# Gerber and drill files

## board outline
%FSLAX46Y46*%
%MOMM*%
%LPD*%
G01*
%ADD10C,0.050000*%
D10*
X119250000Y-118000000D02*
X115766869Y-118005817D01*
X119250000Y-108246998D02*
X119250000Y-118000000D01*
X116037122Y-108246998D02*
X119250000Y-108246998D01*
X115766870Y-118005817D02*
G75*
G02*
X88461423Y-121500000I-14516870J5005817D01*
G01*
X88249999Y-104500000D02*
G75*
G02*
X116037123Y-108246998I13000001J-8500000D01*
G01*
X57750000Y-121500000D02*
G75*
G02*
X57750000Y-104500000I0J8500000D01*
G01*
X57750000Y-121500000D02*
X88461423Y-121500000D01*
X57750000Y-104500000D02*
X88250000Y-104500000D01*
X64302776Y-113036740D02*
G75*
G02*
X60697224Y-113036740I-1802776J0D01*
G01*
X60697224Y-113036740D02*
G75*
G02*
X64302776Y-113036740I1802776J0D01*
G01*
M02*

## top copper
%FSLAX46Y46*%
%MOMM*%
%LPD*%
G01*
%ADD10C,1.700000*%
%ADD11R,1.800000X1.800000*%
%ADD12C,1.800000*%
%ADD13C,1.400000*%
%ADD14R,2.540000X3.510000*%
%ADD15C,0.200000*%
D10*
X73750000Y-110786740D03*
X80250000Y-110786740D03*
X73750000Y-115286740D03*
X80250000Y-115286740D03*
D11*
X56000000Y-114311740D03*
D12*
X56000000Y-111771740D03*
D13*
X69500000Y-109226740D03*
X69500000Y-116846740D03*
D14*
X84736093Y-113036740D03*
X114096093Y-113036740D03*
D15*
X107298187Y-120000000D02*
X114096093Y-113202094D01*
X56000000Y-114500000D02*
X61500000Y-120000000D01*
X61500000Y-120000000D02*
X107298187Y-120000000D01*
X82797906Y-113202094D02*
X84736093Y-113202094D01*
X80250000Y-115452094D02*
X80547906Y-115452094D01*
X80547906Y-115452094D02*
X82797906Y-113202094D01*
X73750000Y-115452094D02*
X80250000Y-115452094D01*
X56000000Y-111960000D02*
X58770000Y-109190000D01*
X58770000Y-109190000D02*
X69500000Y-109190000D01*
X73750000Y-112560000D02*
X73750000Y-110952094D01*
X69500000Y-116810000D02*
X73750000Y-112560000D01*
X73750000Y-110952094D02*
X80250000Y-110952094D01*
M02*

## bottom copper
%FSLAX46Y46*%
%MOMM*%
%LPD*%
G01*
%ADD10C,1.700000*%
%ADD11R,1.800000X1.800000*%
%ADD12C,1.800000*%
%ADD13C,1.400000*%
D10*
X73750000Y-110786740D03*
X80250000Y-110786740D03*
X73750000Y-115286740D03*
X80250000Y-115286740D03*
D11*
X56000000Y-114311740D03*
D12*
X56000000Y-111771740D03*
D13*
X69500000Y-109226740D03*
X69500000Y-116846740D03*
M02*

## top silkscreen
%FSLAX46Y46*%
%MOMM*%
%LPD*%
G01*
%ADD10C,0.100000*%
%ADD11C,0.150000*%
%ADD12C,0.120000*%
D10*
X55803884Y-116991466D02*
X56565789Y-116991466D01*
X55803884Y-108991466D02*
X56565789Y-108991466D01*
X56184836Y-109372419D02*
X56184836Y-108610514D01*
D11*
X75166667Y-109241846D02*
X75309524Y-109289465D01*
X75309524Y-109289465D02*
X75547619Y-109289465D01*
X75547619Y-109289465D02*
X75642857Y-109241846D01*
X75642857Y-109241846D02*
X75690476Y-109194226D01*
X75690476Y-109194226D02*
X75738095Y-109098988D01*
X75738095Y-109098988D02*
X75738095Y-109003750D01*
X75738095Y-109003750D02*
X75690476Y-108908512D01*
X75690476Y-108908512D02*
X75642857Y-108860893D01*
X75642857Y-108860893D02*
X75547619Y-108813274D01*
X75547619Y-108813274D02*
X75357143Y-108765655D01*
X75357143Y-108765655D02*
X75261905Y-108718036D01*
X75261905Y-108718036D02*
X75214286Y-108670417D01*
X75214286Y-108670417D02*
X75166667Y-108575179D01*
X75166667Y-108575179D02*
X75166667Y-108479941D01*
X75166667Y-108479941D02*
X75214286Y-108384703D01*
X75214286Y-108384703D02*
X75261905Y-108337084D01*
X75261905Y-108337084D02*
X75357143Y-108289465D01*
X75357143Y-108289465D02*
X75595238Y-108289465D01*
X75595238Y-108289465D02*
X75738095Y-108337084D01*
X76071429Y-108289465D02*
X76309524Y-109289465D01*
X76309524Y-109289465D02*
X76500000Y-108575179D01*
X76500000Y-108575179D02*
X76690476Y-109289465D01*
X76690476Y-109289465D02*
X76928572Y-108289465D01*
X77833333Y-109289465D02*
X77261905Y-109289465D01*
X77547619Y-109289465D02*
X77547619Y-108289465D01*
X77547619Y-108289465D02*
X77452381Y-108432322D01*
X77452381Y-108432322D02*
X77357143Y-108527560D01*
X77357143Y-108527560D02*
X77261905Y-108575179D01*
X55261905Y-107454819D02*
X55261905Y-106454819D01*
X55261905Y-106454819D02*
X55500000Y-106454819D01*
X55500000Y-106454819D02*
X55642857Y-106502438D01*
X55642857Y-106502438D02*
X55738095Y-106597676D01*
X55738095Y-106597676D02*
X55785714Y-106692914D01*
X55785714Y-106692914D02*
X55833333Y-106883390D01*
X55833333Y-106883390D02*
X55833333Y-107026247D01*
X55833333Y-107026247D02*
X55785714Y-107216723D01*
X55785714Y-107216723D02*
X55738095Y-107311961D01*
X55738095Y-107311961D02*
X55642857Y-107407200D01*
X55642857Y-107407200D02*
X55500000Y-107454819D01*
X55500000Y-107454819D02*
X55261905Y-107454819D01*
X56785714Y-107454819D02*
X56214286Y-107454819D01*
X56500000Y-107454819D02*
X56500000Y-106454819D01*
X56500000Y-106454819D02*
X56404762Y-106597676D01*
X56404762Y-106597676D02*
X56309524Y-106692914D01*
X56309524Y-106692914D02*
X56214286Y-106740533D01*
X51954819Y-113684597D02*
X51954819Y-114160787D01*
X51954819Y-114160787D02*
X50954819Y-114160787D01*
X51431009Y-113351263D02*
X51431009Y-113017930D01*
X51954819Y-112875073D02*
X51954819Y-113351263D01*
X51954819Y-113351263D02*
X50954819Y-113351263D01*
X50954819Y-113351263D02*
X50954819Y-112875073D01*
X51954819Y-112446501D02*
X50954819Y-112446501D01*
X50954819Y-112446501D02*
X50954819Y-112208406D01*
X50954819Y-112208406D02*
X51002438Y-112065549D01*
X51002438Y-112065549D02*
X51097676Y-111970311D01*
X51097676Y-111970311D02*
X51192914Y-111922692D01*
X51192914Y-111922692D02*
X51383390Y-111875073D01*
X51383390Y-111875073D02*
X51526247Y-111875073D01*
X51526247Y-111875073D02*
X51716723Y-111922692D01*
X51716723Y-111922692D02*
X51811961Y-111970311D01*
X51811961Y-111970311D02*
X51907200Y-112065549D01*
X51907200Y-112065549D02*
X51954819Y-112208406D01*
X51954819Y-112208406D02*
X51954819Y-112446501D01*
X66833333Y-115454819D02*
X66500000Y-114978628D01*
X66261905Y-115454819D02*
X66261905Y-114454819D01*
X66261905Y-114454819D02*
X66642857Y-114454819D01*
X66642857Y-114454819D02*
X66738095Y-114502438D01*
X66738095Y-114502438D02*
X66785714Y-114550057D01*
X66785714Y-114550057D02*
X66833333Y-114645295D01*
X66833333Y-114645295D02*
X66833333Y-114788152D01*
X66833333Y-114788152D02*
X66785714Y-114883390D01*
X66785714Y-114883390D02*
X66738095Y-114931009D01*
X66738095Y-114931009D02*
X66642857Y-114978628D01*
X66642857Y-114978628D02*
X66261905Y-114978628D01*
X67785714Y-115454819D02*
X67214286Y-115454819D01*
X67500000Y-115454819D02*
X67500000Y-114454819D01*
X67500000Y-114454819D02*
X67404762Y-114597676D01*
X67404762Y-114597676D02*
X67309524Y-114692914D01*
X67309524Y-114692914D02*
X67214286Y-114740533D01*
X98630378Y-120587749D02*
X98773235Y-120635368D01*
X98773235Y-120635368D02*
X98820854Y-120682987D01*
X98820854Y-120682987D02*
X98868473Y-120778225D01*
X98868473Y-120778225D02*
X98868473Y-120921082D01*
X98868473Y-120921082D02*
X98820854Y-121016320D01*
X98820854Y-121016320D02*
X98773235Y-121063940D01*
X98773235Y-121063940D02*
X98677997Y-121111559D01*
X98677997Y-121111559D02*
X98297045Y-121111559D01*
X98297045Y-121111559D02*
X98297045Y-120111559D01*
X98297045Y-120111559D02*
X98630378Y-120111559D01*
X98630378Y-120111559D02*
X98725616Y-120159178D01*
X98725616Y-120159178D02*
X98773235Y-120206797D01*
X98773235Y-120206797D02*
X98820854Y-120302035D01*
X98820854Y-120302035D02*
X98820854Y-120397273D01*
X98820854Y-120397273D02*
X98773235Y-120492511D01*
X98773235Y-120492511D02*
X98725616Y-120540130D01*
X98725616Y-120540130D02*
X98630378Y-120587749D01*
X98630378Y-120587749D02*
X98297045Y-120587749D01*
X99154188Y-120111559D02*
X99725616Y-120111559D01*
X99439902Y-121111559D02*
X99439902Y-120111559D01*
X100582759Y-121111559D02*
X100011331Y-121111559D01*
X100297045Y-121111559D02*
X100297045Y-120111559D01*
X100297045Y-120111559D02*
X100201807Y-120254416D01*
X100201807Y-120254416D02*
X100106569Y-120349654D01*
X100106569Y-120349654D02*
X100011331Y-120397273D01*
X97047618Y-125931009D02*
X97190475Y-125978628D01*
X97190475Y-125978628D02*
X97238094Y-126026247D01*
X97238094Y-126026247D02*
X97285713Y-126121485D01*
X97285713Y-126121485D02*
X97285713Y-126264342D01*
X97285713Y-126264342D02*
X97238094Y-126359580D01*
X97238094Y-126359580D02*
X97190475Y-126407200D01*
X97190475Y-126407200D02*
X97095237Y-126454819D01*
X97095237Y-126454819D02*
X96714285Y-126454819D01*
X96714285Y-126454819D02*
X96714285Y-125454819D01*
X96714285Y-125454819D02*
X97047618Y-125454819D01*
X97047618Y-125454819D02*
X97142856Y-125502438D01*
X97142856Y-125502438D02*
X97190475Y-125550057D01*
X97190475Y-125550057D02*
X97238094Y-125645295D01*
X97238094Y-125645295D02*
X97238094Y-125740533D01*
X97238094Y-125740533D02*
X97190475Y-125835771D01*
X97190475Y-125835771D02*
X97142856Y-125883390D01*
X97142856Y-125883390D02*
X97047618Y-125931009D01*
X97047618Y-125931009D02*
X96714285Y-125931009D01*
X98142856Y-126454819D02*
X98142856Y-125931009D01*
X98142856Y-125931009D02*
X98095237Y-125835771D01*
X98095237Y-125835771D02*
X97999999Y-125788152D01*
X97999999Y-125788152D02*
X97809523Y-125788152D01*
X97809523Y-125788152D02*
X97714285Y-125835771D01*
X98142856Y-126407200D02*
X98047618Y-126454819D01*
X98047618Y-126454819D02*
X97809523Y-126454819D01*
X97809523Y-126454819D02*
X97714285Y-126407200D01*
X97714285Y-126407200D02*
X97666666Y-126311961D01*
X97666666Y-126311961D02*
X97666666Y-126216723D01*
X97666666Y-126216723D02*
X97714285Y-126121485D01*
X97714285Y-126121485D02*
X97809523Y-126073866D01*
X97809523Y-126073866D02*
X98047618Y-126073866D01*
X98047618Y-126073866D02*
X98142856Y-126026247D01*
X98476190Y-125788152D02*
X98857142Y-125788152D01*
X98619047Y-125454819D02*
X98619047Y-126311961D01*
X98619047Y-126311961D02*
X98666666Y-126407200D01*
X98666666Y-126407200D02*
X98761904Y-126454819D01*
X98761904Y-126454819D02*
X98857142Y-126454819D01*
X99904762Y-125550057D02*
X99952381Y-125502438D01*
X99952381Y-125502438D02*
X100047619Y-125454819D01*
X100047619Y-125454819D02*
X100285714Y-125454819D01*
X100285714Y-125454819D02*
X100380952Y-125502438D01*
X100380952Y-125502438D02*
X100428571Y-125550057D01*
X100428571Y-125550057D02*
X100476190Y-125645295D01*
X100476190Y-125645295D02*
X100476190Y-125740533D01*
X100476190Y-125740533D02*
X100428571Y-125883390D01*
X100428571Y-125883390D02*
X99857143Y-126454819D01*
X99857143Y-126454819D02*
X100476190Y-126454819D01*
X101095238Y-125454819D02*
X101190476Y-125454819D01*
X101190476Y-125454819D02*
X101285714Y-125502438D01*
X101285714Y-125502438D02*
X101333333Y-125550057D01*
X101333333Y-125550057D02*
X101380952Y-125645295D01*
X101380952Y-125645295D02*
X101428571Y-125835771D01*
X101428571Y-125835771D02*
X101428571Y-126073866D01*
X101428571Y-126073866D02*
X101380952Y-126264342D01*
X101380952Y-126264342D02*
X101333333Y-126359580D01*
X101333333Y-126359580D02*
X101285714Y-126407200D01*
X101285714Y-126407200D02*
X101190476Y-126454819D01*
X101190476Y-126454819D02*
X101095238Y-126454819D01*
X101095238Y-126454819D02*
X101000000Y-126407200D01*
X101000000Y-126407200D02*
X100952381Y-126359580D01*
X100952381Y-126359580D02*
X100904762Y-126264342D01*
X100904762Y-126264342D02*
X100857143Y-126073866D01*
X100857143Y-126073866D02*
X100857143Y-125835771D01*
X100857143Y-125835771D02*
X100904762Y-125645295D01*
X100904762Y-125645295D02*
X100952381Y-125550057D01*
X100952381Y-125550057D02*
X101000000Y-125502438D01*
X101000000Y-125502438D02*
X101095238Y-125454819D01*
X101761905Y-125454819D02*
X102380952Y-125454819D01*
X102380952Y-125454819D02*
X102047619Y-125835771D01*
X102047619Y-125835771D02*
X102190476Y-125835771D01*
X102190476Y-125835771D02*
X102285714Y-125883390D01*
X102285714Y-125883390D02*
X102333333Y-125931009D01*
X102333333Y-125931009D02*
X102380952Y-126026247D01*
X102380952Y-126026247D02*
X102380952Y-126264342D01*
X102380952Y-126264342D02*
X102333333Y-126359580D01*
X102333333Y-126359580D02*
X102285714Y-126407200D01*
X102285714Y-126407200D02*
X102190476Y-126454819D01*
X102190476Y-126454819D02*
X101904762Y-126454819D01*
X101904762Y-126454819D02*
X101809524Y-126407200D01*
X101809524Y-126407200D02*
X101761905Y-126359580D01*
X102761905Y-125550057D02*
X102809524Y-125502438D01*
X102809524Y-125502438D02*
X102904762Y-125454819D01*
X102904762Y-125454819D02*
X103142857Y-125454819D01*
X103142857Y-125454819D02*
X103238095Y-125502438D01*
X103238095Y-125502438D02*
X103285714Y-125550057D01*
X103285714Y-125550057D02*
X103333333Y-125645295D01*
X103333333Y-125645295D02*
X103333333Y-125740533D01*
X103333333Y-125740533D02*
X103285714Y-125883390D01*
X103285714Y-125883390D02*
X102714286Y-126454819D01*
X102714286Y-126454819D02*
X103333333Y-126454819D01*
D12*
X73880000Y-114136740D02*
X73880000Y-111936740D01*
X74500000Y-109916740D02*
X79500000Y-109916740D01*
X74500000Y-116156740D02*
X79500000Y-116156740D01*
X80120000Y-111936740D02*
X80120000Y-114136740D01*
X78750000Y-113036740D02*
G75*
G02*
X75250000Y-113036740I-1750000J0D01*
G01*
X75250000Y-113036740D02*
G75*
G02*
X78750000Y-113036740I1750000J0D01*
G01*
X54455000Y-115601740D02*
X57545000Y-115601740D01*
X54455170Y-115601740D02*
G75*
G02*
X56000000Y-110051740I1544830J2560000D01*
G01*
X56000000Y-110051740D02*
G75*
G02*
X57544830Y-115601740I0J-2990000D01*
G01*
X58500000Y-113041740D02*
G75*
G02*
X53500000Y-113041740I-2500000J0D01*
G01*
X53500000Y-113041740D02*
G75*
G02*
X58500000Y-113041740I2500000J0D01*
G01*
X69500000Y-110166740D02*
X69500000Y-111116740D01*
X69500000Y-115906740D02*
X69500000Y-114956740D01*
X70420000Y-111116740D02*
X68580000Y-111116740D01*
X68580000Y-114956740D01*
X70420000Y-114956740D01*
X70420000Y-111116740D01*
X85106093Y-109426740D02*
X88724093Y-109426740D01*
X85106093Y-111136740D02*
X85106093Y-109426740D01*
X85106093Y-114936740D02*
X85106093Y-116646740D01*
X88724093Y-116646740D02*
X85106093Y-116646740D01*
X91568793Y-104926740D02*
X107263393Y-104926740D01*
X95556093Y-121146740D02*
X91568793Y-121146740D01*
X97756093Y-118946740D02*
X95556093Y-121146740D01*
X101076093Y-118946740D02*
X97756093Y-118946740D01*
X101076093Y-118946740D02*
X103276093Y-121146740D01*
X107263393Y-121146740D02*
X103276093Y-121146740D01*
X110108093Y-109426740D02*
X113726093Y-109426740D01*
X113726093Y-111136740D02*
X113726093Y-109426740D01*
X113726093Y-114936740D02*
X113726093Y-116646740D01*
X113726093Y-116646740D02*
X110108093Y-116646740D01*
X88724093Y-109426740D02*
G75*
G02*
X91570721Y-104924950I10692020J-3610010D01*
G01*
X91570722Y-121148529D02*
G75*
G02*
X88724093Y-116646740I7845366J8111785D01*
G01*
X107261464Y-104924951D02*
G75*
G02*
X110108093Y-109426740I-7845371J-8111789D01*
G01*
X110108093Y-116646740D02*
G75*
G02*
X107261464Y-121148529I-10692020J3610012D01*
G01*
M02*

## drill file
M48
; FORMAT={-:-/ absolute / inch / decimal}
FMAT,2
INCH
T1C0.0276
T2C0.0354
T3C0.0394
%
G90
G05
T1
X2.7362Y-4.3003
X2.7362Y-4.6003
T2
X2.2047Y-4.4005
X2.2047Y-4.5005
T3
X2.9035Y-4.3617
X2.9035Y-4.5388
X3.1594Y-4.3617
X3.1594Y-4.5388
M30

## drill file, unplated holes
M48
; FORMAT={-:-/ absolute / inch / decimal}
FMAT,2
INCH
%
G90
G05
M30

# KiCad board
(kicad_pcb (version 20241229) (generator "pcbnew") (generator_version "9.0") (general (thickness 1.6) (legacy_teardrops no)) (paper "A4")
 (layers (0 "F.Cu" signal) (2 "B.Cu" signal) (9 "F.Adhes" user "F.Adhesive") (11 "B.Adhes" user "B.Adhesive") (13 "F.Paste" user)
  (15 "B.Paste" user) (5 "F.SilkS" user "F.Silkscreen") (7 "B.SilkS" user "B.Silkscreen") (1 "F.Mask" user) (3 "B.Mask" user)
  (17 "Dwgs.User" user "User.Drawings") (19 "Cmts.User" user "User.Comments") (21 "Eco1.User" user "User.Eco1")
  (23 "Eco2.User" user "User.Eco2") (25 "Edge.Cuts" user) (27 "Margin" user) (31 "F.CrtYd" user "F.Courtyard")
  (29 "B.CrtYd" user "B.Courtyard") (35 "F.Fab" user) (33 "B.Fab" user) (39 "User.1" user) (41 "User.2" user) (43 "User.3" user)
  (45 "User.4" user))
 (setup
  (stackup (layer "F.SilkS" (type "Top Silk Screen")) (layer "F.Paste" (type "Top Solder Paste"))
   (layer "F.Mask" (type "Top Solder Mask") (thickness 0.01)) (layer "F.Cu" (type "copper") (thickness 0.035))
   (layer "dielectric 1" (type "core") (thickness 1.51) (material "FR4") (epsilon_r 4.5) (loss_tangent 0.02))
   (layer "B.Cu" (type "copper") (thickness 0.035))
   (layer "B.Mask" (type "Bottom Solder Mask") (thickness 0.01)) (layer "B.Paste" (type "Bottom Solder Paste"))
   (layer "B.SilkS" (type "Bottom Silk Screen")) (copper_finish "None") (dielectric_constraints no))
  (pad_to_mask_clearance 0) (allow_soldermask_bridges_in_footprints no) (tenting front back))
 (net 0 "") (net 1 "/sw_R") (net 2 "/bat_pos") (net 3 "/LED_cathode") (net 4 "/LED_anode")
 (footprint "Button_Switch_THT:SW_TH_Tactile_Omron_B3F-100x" (layer "F.Cu") (at 73.75 110.78674)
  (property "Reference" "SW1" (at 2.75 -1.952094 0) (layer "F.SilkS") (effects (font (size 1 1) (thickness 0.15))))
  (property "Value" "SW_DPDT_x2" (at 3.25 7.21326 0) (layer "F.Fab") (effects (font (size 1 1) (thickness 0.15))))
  (fp_line (start 0.13 3.35) (end 0.13 1.15) (stroke (width 0.12) (type solid)) (layer "F.SilkS"))
  (fp_line (start 0.75 -0.87) (end 5.75 -0.87) (stroke (width 0.12) (type solid)) (layer "F.SilkS"))
  (fp_line (start 0.75 5.37) (end 5.75 5.37) (stroke (width 0.12) (type solid)) (layer "F.SilkS"))
  (fp_line (start 6.37 1.15) (end 6.37 3.35) (stroke (width 0.12) (type solid)) (layer "F.SilkS"))
  (fp_circle (center 3.25 2.25) (end 5 2.25) (stroke (width 0.12) (type solid)) (fill no) (layer "F.SilkS"))
  (pad "1" thru_hole circle (at 0 0) (size 1.7 1.7) (drill 1) (layers "*.Cu" "*.Mask") (remove_unused_layers no) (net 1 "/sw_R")
   (thermal_bridge_angle 90))
  (pad "1" thru_hole circle (at 6.5 0) (size 1.7 1.7) (drill 1) (layers "*.Cu" "*.Mask") (remove_unused_layers no) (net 1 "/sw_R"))
  (pad "2" thru_hole circle (at 0 4.5) (size 1.7 1.7) (drill 1) (layers "*.Cu" "*.Mask") (remove_unused_layers no) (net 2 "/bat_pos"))
  (pad "2" thru_hole circle (at 6.5 4.5) (size 1.7 1.7) (drill 1) (layers "*.Cu" "*.Mask") (remove_unused_layers no) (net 2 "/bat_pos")))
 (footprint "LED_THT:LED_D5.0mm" (layer "F.Cu") (at 56 114.31174 90)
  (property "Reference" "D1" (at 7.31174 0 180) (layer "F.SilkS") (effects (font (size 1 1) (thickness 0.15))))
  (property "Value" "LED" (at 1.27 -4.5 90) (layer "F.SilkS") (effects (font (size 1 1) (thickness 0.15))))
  (fp_line (start -1.29 -1.545) (end -1.29 1.545) (stroke (width 0.12) (type solid)) (layer "F.SilkS"))
  (fp_arc (start -1.29 -1.54483) (mid 2.071779 -2.880495) (end 4.26 0) (stroke (width 0.12) (type solid)) (layer "F.SilkS"))
  (fp_arc (start 4.26 0) (mid 2.071779 2.880495) (end -1.29 1.54483) (stroke (width 0.12) (type solid)) (layer "F.SilkS"))
  (fp_circle (center 1.27 0) (end 3.77 0) (stroke (width 0.12) (type solid)) (fill no) (layer "F.SilkS"))
  (pad "1" thru_hole rect (at 0 0 90) (size 1.8 1.8) (drill 0.9) (layers "*.Cu" "*.Mask") (remove_unused_layers no) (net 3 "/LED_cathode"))
  (pad "2" thru_hole circle (at 2.54 0 90) (size 1.8 1.8) (drill 0.9) (layers "*.Cu" "*.Mask") (remove_unused_layers no)
   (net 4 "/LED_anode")))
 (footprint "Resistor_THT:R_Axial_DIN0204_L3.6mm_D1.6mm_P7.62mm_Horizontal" (layer "F.Cu") (at 69.5 109.22674 -90)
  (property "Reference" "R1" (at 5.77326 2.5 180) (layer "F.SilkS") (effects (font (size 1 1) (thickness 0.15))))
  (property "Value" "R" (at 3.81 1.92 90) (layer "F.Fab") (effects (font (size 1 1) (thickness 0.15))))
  (fp_line (start 0.94 0) (end 1.89 0) (stroke (width 0.12) (type solid)) (layer "F.SilkS"))
  (fp_line (start 6.68 0) (end 5.73 0) (stroke (width 0.12) (type solid)) (layer "F.SilkS"))
  (fp_rect (start 1.89 -0.92) (end 5.73 0.92) (stroke (width 0.12) (type solid)) (fill no) (layer "F.SilkS"))
  (pad "1" thru_hole circle (at 0 0 270) (size 1.4 1.4) (drill 0.7) (layers "*.Cu" "*.Mask") (remove_unused_layers no) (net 4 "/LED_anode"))
  (pad "2" thru_hole circle (at 7.62 0 270) (size 1.4 1.4) (drill 0.7) (layers "*.Cu" "*.Mask") (remove_unused_layers no) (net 1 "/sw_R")))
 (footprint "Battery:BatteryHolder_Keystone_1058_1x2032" (layer "F.Cu") (at 99.416093 113.03674)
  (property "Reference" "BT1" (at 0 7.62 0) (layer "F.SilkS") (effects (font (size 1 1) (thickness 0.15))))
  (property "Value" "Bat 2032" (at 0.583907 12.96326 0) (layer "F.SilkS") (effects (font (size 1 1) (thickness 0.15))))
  (fp_line (start -14.31 -3.61) (end -10.692 -3.61) (stroke (width 0.12) (type solid)) (layer "F.SilkS"))
  (fp_line (start -14.31 -1.9) (end -14.31 -3.61) (stroke (width 0.12) (type solid)) (layer "F.SilkS"))
  (fp_line (start -14.31 1.9) (end -14.31 3.61) (stroke (width 0.12) (type solid)) (layer "F.SilkS"))
  (fp_line (start -10.692 3.61) (end -14.31 3.61) (stroke (width 0.12) (type solid)) (layer "F.SilkS"))
  (fp_line (start -7.8473 -8.11) (end 7.8473 -8.11) (stroke (width 0.12) (type solid)) (layer "F.SilkS"))
  (fp_line (start -3.86 8.11) (end -7.8473 8.11) (stroke (width 0.12) (type solid)) (layer "F.SilkS"))
  (fp_line (start -1.66 5.91) (end -3.86 8.11) (stroke (width 0.12) (type solid)) (layer "F.SilkS"))
  (fp_line (start 1.66 5.91) (end -1.66 5.91) (stroke (width 0.12) (type solid)) (layer "F.SilkS"))
  (fp_line (start 1.66 5.91) (end 3.86 8.11) (stroke (width 0.12) (type solid)) (layer "F.SilkS"))
  (fp_line (start 7.8473 8.11) (end 3.86 8.11) (stroke (width 0.12) (type solid)) (layer "F.SilkS"))
  (fp_line (start 10.692 -3.61) (end 14.31 -3.61) (stroke (width 0.12) (type solid)) (layer "F.SilkS"))
  (fp_line (start 14.31 -1.9) (end 14.31 -3.61) (stroke (width 0.12) (type solid)) (layer "F.SilkS"))
  (fp_line (start 14.31 1.9) (end 14.31 3.61) (stroke (width 0.12) (type solid)) (layer "F.SilkS"))
  (fp_line (start 14.31 3.61) (end 10.692 3.61) (stroke (width 0.12) (type solid)) (layer "F.SilkS"))
  (fp_arc (start -10.692 -3.61) (mid -9.538084 -6.031244) (end -7.845371 -8.111789) (stroke (width 0.12) (type solid)) (layer "F.SilkS"))
  (fp_arc (start -7.845371 8.111789) (mid -9.538085 6.031244) (end -10.692 3.61) (stroke (width 0.12) (type solid)) (layer "F.SilkS"))
  (fp_arc (start 7.845371 -8.111789) (mid 9.538085 -6.031244) (end 10.692 -3.61) (stroke (width 0.12) (type solid)) (layer "F.SilkS"))
  (fp_arc (start 10.692 3.61) (mid 9.538084 6.031244) (end 7.845371 8.111789) (stroke (width 0.12) (type solid)) (layer "F.SilkS"))
  (pad "1" smd rect (at -14.68 0) (size 2.54 3.51) (layers "F.Cu" "F.Mask" "F.Paste") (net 2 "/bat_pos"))
  (pad "2" smd rect (at 14.68 0) (size 2.54 3.51) (layers "F.Cu" "F.Mask" "F.Paste") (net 3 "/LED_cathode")))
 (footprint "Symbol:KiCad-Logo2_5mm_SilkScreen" (layer "B.Cu") (at 99 112.5 180)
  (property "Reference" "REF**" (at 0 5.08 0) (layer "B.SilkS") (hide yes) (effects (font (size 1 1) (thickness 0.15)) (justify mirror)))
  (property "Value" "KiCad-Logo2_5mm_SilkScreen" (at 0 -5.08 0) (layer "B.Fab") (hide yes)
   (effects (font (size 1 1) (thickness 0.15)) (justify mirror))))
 (gr_line (start 116.037122 108.246998) (end 119.25 108.246998) (stroke (width 0.05) (type default)) (locked yes) (layer "Edge.Cuts"))
 (gr_arc (start 88.249999 104.5) (mid 103.32568 97.607093) (end 116.037122 108.246998) (stroke (width 0.05) (type default)) (locked yes)
  (layer "Edge.Cuts"))
 (gr_line (start 57.75 121.5) (end 88.461423 121.5) (stroke (width 0.05) (type default)) (locked yes) (layer "Edge.Cuts"))
 (gr_arc (start 57.75 121.5) (mid 49.25 113) (end 57.75 104.5) (stroke (width 0.05) (type default)) (locked yes) (layer "Edge.Cuts"))
 (gr_line (start 57.75 104.5) (end 88.25 104.5) (stroke (width 0.05) (type default)) (locked yes) (layer "Edge.Cuts"))
 (gr_arc (start 115.76687 118.005817) (mid 103.199122 128.231502) (end 88.461423 121.5) (stroke (width 0.05) (type default)) (locked yes)
  (layer "Edge.Cuts"))
 (gr_line (start 119.25 118) (end 115.766869 118.005817) (stroke (width 0.05) (type default)) (locked yes) (layer "Edge.Cuts"))
 (gr_line (start 119.25 108.246998) (end 119.25 118) (stroke (width 0.05) (type default)) (locked yes) (layer "Edge.Cuts"))
 (gr_circle (center 62.5 113.03674) (end 64 114.03674) (stroke (width 0.05) (type default)) (fill no) (layer "Edge.Cuts"))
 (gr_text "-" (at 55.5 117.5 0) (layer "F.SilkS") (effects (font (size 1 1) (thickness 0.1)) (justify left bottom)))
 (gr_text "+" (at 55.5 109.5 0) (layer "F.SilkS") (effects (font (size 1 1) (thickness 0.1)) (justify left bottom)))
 (segment (start 107.298187 120) (end 114.096093 113.202094) (width 0.2) (layer "F.Cu") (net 3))
 (segment (start 56 114.5) (end 61.5 120) (width 0.2) (layer "F.Cu") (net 3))
 (segment (start 61.5 120) (end 107.298187 120) (width 0.2) (layer "F.Cu") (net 3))
 (segment (start 82.797906 113.202094) (end 84.736093 113.202094) (width 0.2) (layer "F.Cu") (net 2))
 (segment (start 80.25 115.452094) (end 80.547906 115.452094) (width 0.2) (layer "F.Cu") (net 2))
 (segment (start 80.547906 115.452094) (end 82.797906 113.202094) (width 0.2) (layer "F.Cu") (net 2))
 (segment (start 73.75 115.452094) (end 80.25 115.452094) (width 0.2) (layer "F.Cu") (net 2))
 (segment (start 56 111.96) (end 58.77 109.19) (width 0.2) (layer "F.Cu") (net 4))
 (segment (start 58.77 109.19) (end 69.5 109.19) (width 0.2) (layer "F.Cu") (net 4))
 (segment (start 73.75 112.56) (end 73.75 110.952094) (width 0.2) (layer "F.Cu") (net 1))
 (segment (start 69.5 116.81) (end 73.75 112.56) (width 0.2) (layer "F.Cu") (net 1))
 (segment (start 73.75 110.952094) (end 80.25 110.952094) (width 0.2) (layer "F.Cu") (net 1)))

